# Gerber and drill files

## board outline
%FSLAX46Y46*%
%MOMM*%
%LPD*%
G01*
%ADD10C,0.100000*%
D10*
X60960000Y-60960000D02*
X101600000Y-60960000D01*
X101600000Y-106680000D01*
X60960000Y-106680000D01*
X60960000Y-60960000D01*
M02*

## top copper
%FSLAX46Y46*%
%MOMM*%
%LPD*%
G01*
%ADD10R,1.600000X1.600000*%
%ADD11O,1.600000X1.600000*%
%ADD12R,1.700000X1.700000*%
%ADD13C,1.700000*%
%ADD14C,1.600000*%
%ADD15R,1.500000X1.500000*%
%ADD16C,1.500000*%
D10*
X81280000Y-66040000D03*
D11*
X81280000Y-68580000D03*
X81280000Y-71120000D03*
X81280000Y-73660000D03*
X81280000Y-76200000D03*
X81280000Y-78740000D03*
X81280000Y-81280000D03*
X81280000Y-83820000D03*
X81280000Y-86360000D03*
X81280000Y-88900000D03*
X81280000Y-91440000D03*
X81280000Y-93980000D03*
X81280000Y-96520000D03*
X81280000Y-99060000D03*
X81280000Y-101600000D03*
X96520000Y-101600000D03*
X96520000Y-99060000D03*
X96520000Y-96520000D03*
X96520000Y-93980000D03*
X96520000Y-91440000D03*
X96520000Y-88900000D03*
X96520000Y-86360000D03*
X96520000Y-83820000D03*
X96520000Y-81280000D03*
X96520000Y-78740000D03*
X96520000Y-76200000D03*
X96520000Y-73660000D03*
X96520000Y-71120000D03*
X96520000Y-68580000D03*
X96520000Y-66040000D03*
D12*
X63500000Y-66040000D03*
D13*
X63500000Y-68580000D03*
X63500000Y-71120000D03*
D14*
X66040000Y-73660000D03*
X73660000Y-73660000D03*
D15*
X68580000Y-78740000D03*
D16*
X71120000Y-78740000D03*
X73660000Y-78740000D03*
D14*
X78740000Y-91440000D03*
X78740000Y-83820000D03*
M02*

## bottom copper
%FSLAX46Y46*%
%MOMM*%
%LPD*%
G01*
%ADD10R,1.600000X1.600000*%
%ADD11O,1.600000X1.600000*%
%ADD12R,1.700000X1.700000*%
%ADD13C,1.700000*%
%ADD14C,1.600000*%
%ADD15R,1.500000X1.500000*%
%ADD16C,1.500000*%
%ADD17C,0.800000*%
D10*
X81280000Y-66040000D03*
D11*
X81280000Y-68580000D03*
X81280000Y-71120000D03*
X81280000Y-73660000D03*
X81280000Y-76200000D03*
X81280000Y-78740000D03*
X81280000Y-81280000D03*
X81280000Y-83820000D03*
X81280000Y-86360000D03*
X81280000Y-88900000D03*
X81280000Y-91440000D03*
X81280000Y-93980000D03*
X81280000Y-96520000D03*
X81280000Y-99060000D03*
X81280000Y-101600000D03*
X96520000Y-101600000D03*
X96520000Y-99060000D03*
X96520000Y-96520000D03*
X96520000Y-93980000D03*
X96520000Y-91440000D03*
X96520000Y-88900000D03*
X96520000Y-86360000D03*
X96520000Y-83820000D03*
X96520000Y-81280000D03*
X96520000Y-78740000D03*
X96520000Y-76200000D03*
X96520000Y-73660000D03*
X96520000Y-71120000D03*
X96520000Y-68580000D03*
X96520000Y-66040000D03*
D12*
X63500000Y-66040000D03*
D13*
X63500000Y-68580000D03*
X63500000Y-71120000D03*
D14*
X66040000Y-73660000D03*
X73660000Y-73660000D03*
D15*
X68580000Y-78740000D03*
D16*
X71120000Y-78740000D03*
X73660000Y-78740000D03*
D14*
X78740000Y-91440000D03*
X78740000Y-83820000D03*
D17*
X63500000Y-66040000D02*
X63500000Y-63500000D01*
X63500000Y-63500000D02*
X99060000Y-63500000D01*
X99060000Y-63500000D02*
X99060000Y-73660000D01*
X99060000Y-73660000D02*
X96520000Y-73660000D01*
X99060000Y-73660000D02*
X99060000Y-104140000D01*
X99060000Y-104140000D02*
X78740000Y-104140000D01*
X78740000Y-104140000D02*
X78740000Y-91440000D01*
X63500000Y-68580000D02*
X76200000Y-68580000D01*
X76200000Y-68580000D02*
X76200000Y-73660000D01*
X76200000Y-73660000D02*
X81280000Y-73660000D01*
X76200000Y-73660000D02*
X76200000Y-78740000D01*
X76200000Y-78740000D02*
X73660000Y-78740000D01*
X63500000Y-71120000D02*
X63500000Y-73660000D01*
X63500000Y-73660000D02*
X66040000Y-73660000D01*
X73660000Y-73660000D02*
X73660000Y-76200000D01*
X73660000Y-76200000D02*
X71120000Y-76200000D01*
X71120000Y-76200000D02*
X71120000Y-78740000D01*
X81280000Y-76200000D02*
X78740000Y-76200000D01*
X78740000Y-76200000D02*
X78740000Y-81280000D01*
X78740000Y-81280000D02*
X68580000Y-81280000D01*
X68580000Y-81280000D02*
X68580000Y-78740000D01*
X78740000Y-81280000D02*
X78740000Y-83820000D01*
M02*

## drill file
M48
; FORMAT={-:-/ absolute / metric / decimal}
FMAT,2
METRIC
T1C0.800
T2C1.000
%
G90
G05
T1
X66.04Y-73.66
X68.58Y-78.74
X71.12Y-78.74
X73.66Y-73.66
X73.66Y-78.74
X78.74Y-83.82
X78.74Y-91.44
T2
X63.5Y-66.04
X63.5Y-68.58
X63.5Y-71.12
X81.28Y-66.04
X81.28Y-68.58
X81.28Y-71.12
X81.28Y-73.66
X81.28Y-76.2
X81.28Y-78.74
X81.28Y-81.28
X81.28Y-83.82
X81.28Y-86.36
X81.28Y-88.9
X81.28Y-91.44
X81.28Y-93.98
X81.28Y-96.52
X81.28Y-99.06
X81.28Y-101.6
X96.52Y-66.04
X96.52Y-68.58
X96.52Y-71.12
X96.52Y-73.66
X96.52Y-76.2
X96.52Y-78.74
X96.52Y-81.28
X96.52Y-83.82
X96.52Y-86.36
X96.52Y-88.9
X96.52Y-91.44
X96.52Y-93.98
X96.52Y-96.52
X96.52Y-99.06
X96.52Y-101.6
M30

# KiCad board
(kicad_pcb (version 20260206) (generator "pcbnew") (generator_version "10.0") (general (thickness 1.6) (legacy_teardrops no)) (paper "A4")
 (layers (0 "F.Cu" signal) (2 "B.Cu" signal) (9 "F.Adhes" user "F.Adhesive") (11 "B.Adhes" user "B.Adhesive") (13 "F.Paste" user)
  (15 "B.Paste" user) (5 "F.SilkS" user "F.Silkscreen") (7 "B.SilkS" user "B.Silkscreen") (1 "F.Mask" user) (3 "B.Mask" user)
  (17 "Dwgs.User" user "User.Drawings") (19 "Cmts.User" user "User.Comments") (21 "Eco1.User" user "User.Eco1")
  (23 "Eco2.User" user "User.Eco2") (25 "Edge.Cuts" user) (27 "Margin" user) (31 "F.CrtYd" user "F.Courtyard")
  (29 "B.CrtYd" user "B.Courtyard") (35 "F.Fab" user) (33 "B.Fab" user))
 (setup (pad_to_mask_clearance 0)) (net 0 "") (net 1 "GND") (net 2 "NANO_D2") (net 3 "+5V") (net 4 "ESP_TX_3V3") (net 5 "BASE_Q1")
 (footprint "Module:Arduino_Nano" (layer "F.Cu") (at 81.280 66.040 0)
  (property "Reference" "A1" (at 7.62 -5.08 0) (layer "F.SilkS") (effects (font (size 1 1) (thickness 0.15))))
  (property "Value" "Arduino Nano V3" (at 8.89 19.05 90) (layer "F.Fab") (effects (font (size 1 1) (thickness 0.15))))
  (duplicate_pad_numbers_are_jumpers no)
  (pad "1" thru_hole rect (at 0 0) (size 1.6 1.6) (drill 1) (layers "*.Cu" "*.Mask") (remove_unused_layers no))
  (pad "2" thru_hole oval (at 0 2.54) (size 1.6 1.6) (drill 1) (layers "*.Cu" "*.Mask") (remove_unused_layers no))
  (pad "3" thru_hole oval (at 0 5.08) (size 1.6 1.6) (drill 1) (layers "*.Cu" "*.Mask") (remove_unused_layers no))
  (pad "4" thru_hole oval (at 0 7.62) (size 1.6 1.6) (drill 1) (layers "*.Cu" "*.Mask") (remove_unused_layers no) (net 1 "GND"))
  (pad "5" thru_hole oval (at 0 10.16) (size 1.6 1.6) (drill 1) (layers "*.Cu" "*.Mask") (remove_unused_layers no) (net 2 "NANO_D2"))
  (pad "6" thru_hole oval (at 0 12.7) (size 1.6 1.6) (drill 1) (layers "*.Cu" "*.Mask") (remove_unused_layers no))
  (pad "7" thru_hole oval (at 0 15.24) (size 1.6 1.6) (drill 1) (layers "*.Cu" "*.Mask") (remove_unused_layers no))
  (pad "8" thru_hole oval (at 0 17.78) (size 1.6 1.6) (drill 1) (layers "*.Cu" "*.Mask") (remove_unused_layers no))
  (pad "9" thru_hole oval (at 0 20.32) (size 1.6 1.6) (drill 1) (layers "*.Cu" "*.Mask") (remove_unused_layers no))
  (pad "10" thru_hole oval (at 0 22.86) (size 1.6 1.6) (drill 1) (layers "*.Cu" "*.Mask") (remove_unused_layers no))
  (pad "11" thru_hole oval (at 0 25.4) (size 1.6 1.6) (drill 1) (layers "*.Cu" "*.Mask") (remove_unused_layers no))
  (pad "12" thru_hole oval (at 0 27.94) (size 1.6 1.6) (drill 1) (layers "*.Cu" "*.Mask") (remove_unused_layers no))
  (pad "13" thru_hole oval (at 0 30.48) (size 1.6 1.6) (drill 1) (layers "*.Cu" "*.Mask") (remove_unused_layers no))
  (pad "14" thru_hole oval (at 0 33.02) (size 1.6 1.6) (drill 1) (layers "*.Cu" "*.Mask") (remove_unused_layers no))
  (pad "15" thru_hole oval (at 0 35.56) (size 1.6 1.6) (drill 1) (layers "*.Cu" "*.Mask") (remove_unused_layers no))
  (pad "16" thru_hole oval (at 15.24 35.56) (size 1.6 1.6) (drill 1) (layers "*.Cu" "*.Mask") (remove_unused_layers no))
  (pad "17" thru_hole oval (at 15.24 33.02) (size 1.6 1.6) (drill 1) (layers "*.Cu" "*.Mask") (remove_unused_layers no))
  (pad "18" thru_hole oval (at 15.24 30.48) (size 1.6 1.6) (drill 1) (layers "*.Cu" "*.Mask") (remove_unused_layers no))
  (pad "19" thru_hole oval (at 15.24 27.94) (size 1.6 1.6) (drill 1) (layers "*.Cu" "*.Mask") (remove_unused_layers no))
  (pad "20" thru_hole oval (at 15.24 25.4) (size 1.6 1.6) (drill 1) (layers "*.Cu" "*.Mask") (remove_unused_layers no))
  (pad "21" thru_hole oval (at 15.24 22.86) (size 1.6 1.6) (drill 1) (layers "*.Cu" "*.Mask") (remove_unused_layers no))
  (pad "22" thru_hole oval (at 15.24 20.32) (size 1.6 1.6) (drill 1) (layers "*.Cu" "*.Mask") (remove_unused_layers no))
  (pad "23" thru_hole oval (at 15.24 17.78) (size 1.6 1.6) (drill 1) (layers "*.Cu" "*.Mask") (remove_unused_layers no))
  (pad "24" thru_hole oval (at 15.24 15.24) (size 1.6 1.6) (drill 1) (layers "*.Cu" "*.Mask") (remove_unused_layers no))
  (pad "25" thru_hole oval (at 15.24 12.7) (size 1.6 1.6) (drill 1) (layers "*.Cu" "*.Mask") (remove_unused_layers no))
  (pad "26" thru_hole oval (at 15.24 10.16) (size 1.6 1.6) (drill 1) (layers "*.Cu" "*.Mask") (remove_unused_layers no))
  (pad "27" thru_hole oval (at 15.24 7.62) (size 1.6 1.6) (drill 1) (layers "*.Cu" "*.Mask") (remove_unused_layers no) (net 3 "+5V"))
  (pad "28" thru_hole oval (at 15.24 5.08) (size 1.6 1.6) (drill 1) (layers "*.Cu" "*.Mask") (remove_unused_layers no))
  (pad "29" thru_hole oval (at 15.24 2.54) (size 1.6 1.6) (drill 1) (layers "*.Cu" "*.Mask") (remove_unused_layers no) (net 1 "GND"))
  (pad "30" thru_hole oval (at 15.24 0) (size 1.6 1.6) (drill 1) (layers "*.Cu" "*.Mask") (remove_unused_layers no)))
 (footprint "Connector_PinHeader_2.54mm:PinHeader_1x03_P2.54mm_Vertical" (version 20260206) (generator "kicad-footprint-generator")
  (layer "F.Cu") (at 63.500 66.040 0)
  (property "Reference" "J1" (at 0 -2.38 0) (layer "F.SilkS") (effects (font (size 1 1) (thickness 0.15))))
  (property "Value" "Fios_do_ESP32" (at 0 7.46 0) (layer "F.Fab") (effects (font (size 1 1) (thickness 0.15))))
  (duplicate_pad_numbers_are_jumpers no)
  (pad "1" thru_hole rect (at 0 0) (size 1.7 1.7) (drill 1) (layers "*.Cu" "*.Mask") (remove_unused_layers no) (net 3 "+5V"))
  (pad "2" thru_hole circle (at 0 2.54) (size 1.7 1.7) (drill 1) (layers "*.Cu" "*.Mask") (remove_unused_layers no) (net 1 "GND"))
  (pad "3" thru_hole circle (at 0 5.08) (size 1.7 1.7) (drill 1) (layers "*.Cu" "*.Mask") (remove_unused_layers no) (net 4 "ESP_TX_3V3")))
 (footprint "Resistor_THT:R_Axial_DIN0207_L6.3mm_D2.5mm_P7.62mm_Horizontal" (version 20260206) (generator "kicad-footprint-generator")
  (layer "F.Cu") (at 66.040 73.660 0)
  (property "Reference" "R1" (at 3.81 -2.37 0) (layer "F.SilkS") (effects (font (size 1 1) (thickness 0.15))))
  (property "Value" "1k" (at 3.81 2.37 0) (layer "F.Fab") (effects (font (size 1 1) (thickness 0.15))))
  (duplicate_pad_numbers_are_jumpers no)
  (pad "1" thru_hole circle (at 0 0) (size 1.6 1.6) (drill 0.8) (layers "*.Cu" "*.Mask") (remove_unused_layers no) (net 4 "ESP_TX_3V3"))
  (pad "2" thru_hole circle (at 7.62 0) (size 1.6 1.6) (drill 0.8) (layers "*.Cu" "*.Mask") (remove_unused_layers no) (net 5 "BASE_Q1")))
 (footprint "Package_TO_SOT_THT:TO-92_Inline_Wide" (layer "F.Cu") (at 68.580 78.740 0)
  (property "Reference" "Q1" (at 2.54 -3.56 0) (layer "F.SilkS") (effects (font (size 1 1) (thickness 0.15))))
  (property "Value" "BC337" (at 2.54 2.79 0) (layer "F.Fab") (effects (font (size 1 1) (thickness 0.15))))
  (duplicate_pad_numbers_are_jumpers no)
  (pad "1" thru_hole rect (at 0 0) (size 1.5 1.5) (drill 0.8) (layers "*.Cu" "*.Mask") (remove_unused_layers no) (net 2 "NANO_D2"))
  (pad "2" thru_hole circle (at 2.54 0) (size 1.5 1.5) (drill 0.8) (layers "*.Cu" "*.Mask") (remove_unused_layers no) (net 5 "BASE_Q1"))
  (pad "3" thru_hole circle (at 5.08 0) (size 1.5 1.5) (drill 0.8) (layers "*.Cu" "*.Mask") (remove_unused_layers no) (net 1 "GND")))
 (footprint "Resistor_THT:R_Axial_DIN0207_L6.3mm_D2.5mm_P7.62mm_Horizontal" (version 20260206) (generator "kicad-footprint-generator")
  (layer "F.Cu") (at 78.740 91.440 90)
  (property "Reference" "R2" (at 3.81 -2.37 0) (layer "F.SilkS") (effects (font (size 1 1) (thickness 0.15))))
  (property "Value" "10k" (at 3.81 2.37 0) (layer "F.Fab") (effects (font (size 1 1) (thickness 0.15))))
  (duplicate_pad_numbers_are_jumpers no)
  (pad "1" thru_hole circle (at 0 0) (size 1.6 1.6) (drill 0.8) (layers "*.Cu" "*.Mask") (remove_unused_layers no) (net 3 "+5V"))
  (pad "2" thru_hole circle (at 7.62 0) (size 1.6 1.6) (drill 0.8) (layers "*.Cu" "*.Mask") (remove_unused_layers no) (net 2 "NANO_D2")))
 (segment (start 63.500 66.040) (end 63.500 63.500) (width 0.8) (layer "B.Cu") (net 3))
 (segment (start 63.500 63.500) (end 99.060 63.500) (width 0.8) (layer "B.Cu") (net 3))
 (segment (start 99.060 63.500) (end 99.060 73.660) (width 0.8) (layer "B.Cu") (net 3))
 (segment (start 99.060 73.660) (end 96.520 73.660) (width 0.8) (layer "B.Cu") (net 3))
 (segment (start 99.060 73.660) (end 99.060 104.140) (width 0.8) (layer "B.Cu") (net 3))
 (segment (start 99.060 104.140) (end 78.740 104.140) (width 0.8) (layer "B.Cu") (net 3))
 (segment (start 78.740 104.140) (end 78.740 91.440) (width 0.8) (layer "B.Cu") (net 3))
 (segment (start 63.500 68.580) (end 76.200 68.580) (width 0.8) (layer "B.Cu") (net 1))
 (segment (start 76.200 68.580) (end 76.200 73.660) (width 0.8) (layer "B.Cu") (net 1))
 (segment (start 76.200 73.660) (end 81.280 73.660) (width 0.8) (layer "B.Cu") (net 1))
 (segment (start 76.200 73.660) (end 76.200 78.740) (width 0.8) (layer "B.Cu") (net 1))
 (segment (start 76.200 78.740) (end 73.660 78.740) (width 0.8) (layer "B.Cu") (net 1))
 (segment (start 63.500 71.120) (end 63.500 73.660) (width 0.8) (layer "B.Cu") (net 4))
 (segment (start 63.500 73.660) (end 66.040 73.660) (width 0.8) (layer "B.Cu") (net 4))
 (segment (start 73.660 73.660) (end 73.660 76.200) (width 0.8) (layer "B.Cu") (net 5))
 (segment (start 73.660 76.200) (end 71.120 76.200) (width 0.8) (layer "B.Cu") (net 5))
 (segment (start 71.120 76.200) (end 71.120 78.740) (width 0.8) (layer "B.Cu") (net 5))
 (segment (start 81.280 76.200) (end 78.740 76.200) (width 0.8) (layer "B.Cu") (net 2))
 (segment (start 78.740 76.200) (end 78.740 81.280) (width 0.8) (layer "B.Cu") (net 2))
 (segment (start 78.740 81.280) (end 68.580 81.280) (width 0.8) (layer "B.Cu") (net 2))
 (segment (start 68.580 81.280) (end 68.580 78.740) (width 0.8) (layer "B.Cu") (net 2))
 (segment (start 78.740 81.280) (end 78.740 83.820) (width 0.8) (layer "B.Cu") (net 2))
 (gr_rect (start 60.960 60.960) (end 101.600 106.680) (stroke (width 0.1) (type default)) (fill no) (layer "Edge.Cuts")))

